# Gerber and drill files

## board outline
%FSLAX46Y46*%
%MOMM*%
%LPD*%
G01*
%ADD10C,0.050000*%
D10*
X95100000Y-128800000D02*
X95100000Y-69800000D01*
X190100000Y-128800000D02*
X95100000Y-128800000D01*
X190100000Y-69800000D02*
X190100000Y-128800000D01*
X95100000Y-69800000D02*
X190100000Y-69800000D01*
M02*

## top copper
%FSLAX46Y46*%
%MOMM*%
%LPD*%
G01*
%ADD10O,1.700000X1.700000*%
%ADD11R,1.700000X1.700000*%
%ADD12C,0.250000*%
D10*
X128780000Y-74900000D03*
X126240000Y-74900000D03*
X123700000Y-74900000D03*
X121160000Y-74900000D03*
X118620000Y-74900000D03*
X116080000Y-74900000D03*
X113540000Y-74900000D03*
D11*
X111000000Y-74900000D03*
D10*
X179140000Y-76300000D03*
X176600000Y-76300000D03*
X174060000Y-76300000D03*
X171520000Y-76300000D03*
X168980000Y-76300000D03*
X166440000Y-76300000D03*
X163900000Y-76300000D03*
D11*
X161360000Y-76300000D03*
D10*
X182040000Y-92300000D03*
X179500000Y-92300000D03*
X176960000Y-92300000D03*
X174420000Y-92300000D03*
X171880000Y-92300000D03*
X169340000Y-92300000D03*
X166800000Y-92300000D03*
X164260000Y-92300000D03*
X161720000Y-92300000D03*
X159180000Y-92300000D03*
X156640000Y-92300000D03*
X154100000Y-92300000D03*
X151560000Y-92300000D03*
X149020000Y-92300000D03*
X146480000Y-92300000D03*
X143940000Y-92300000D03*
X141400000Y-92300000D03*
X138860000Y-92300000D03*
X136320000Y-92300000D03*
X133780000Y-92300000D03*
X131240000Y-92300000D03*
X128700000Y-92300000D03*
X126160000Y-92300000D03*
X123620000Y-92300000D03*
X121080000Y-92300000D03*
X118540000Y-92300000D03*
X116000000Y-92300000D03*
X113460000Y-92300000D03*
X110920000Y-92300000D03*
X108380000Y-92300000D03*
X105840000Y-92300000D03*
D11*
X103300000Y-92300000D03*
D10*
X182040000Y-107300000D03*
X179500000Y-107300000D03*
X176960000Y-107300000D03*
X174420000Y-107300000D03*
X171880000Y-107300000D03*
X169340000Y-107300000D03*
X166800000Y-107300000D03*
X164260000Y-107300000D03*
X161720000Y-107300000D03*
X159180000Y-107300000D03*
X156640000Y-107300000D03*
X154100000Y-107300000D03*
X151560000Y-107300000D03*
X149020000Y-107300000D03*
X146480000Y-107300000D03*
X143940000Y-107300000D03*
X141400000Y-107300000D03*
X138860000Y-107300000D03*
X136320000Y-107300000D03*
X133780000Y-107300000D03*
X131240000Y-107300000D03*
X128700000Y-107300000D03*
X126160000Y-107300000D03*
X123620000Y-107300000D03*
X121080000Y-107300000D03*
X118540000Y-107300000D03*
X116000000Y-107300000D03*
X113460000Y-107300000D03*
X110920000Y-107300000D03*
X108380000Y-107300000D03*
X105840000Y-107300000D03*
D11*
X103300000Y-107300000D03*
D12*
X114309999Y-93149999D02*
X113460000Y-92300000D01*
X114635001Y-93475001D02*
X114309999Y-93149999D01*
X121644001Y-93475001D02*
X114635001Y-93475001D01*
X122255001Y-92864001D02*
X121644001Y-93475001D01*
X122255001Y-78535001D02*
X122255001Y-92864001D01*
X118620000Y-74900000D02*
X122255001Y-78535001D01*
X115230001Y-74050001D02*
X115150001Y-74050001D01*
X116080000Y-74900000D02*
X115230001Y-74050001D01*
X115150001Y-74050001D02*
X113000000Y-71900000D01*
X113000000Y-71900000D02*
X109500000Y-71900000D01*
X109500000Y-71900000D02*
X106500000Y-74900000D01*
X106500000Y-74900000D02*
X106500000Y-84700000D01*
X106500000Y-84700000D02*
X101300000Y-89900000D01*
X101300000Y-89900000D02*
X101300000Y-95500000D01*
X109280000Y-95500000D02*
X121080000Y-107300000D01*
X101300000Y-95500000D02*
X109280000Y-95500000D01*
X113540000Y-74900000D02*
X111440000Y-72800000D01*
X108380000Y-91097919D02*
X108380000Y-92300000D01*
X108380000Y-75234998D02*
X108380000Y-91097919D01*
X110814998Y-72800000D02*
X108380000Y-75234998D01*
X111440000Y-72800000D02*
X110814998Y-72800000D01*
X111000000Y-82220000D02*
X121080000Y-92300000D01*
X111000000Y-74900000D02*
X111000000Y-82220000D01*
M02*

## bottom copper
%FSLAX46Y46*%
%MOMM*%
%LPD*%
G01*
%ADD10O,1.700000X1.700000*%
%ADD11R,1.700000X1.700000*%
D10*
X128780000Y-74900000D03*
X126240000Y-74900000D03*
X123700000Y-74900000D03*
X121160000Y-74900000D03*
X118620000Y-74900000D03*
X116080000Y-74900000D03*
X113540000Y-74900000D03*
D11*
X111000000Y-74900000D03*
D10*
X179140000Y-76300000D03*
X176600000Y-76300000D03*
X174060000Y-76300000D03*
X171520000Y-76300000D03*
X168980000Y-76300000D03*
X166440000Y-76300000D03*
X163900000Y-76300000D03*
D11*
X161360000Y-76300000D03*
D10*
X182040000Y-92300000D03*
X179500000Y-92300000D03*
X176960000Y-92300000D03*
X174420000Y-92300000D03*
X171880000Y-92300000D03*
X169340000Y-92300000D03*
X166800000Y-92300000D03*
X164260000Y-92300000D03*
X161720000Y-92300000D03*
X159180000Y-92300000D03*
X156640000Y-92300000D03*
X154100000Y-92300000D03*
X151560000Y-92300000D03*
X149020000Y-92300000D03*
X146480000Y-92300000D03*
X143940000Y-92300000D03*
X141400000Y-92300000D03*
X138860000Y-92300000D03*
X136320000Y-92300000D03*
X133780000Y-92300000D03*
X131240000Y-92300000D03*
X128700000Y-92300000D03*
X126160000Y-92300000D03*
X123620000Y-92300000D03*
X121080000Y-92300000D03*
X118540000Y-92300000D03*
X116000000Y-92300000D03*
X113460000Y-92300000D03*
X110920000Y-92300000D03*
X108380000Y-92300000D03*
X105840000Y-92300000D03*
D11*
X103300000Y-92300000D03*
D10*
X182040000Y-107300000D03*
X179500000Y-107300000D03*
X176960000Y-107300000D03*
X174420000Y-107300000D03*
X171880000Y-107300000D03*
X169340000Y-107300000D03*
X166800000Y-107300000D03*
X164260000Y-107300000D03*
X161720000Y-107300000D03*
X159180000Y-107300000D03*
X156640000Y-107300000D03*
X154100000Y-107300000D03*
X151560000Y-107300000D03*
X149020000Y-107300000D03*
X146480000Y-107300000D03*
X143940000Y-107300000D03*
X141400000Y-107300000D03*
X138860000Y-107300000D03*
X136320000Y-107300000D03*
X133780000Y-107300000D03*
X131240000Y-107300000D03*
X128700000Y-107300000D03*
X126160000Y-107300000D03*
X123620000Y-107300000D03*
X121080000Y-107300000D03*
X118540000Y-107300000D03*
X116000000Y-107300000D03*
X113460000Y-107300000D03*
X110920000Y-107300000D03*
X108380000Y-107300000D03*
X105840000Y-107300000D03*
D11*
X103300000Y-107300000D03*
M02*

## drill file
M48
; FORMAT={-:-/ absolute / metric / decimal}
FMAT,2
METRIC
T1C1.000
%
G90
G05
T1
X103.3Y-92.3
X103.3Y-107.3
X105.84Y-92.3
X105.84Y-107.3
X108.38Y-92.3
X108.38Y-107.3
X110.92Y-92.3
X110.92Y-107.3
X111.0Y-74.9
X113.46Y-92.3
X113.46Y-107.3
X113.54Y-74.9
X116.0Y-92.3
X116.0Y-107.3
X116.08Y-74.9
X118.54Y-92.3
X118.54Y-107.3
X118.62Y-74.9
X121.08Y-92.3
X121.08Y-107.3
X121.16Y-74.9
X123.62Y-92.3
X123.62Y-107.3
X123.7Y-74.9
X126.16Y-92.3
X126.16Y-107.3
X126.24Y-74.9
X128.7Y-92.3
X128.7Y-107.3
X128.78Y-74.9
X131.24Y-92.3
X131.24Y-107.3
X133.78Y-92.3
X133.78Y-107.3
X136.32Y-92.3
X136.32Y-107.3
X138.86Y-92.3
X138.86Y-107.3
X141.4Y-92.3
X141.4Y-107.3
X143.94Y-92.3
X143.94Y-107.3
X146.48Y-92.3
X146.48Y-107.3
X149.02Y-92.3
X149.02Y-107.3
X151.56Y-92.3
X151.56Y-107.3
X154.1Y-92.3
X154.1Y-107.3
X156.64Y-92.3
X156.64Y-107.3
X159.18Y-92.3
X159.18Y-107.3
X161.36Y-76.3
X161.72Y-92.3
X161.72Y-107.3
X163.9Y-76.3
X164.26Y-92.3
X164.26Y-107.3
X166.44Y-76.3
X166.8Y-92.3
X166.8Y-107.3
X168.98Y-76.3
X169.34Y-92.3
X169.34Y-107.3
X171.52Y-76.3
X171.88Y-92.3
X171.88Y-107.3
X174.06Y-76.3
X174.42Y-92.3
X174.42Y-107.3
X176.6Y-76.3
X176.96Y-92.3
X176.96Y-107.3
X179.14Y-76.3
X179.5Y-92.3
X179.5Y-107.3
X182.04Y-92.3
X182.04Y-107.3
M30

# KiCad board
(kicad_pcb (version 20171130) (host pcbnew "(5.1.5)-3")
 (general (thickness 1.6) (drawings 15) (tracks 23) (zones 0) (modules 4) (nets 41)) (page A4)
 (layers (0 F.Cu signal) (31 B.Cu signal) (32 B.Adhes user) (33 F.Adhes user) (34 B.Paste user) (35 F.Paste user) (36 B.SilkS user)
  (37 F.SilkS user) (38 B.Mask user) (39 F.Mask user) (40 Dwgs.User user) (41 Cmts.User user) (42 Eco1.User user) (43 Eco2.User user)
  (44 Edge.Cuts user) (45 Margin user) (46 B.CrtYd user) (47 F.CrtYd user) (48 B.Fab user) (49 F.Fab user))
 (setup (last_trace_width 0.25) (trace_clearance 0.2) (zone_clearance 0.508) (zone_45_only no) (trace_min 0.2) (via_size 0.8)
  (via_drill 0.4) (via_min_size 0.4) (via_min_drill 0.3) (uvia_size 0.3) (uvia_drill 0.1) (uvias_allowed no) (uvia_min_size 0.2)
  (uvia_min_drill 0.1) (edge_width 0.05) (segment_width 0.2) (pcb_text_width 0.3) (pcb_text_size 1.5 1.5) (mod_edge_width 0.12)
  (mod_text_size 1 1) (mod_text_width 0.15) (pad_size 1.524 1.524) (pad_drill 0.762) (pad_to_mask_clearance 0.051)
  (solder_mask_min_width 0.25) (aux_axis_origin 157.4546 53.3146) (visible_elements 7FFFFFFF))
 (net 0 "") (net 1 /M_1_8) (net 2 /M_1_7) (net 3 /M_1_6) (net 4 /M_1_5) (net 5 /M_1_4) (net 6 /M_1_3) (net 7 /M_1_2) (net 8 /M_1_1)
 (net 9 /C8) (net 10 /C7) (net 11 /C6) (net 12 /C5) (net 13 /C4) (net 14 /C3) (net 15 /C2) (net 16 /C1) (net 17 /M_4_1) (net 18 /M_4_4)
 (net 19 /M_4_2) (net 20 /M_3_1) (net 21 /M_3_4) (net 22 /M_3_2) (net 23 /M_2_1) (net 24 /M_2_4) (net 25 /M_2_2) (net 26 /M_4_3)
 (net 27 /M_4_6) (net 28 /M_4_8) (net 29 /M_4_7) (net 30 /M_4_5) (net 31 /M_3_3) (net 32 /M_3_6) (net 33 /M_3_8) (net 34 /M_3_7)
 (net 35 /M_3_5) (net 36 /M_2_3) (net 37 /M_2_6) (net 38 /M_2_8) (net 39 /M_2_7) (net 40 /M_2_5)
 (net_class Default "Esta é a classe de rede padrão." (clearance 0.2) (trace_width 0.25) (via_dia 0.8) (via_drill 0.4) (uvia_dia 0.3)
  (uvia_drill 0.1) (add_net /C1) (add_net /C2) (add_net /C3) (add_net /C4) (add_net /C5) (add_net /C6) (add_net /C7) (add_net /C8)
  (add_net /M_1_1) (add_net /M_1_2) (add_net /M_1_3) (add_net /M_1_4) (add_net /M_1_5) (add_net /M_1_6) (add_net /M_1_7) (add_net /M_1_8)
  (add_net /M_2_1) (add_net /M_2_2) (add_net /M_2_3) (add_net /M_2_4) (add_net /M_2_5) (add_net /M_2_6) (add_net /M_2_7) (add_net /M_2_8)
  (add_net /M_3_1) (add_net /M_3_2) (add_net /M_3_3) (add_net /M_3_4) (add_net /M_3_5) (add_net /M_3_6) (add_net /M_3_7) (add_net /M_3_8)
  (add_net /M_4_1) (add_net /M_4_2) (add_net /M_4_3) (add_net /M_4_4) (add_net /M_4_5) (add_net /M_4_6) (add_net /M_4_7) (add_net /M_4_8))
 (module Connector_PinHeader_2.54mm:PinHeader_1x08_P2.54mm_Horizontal (layer F.Cu) (at 111 74.9 90)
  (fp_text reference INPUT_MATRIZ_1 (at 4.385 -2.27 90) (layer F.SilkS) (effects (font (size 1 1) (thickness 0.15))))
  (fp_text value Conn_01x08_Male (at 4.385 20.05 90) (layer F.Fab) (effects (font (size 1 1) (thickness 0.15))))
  (pad 8 thru_hole oval (at 0 17.78 90) (size 1.7 1.7) (drill 1) (layers *.Cu *.Mask) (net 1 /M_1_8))
  (pad 7 thru_hole oval (at 0 15.24 90) (size 1.7 1.7) (drill 1) (layers *.Cu *.Mask) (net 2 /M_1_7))
  (pad 6 thru_hole oval (at 0 12.7 90) (size 1.7 1.7) (drill 1) (layers *.Cu *.Mask) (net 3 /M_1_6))
  (pad 5 thru_hole oval (at 0 10.16 90) (size 1.7 1.7) (drill 1) (layers *.Cu *.Mask) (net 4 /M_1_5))
  (pad 4 thru_hole oval (at 0 7.62 90) (size 1.7 1.7) (drill 1) (layers *.Cu *.Mask) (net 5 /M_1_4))
  (pad 3 thru_hole oval (at 0 5.08 90) (size 1.7 1.7) (drill 1) (layers *.Cu *.Mask) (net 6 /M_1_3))
  (pad 2 thru_hole oval (at 0 2.54 90) (size 1.7 1.7) (drill 1) (layers *.Cu *.Mask) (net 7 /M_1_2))
  (pad 1 thru_hole rect (at 0 0 90) (size 1.7 1.7) (drill 1) (layers *.Cu *.Mask) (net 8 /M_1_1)))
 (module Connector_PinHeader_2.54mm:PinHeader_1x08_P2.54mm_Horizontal (layer F.Cu) (at 161.36 76.3 90)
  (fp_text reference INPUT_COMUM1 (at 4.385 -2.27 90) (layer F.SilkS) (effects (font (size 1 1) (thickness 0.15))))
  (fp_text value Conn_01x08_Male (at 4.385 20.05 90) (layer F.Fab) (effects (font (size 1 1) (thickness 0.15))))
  (pad 8 thru_hole oval (at 0 17.78 90) (size 1.7 1.7) (drill 1) (layers *.Cu *.Mask) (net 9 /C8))
  (pad 7 thru_hole oval (at 0 15.24 90) (size 1.7 1.7) (drill 1) (layers *.Cu *.Mask) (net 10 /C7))
  (pad 6 thru_hole oval (at 0 12.7 90) (size 1.7 1.7) (drill 1) (layers *.Cu *.Mask) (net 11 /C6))
  (pad 5 thru_hole oval (at 0 10.16 90) (size 1.7 1.7) (drill 1) (layers *.Cu *.Mask) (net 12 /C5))
  (pad 4 thru_hole oval (at 0 7.62 90) (size 1.7 1.7) (drill 1) (layers *.Cu *.Mask) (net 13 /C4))
  (pad 3 thru_hole oval (at 0 5.08 90) (size 1.7 1.7) (drill 1) (layers *.Cu *.Mask) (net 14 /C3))
  (pad 2 thru_hole oval (at 0 2.54 90) (size 1.7 1.7) (drill 1) (layers *.Cu *.Mask) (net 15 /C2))
  (pad 1 thru_hole rect (at 0 0 90) (size 1.7 1.7) (drill 1) (layers *.Cu *.Mask) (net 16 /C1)))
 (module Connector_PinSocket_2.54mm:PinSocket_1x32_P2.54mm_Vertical (layer F.Cu) (at 103.3 92.3 90)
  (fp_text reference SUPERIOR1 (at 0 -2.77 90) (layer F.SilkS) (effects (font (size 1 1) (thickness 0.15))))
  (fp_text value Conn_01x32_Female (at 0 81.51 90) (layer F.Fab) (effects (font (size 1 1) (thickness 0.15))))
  (pad 32 thru_hole oval (at 0 78.74 90) (size 1.7 1.7) (drill 1) (layers *.Cu *.Mask) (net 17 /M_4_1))
  (pad 31 thru_hole oval (at 0 76.2 90) (size 1.7 1.7) (drill 1) (layers *.Cu *.Mask) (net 13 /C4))
  (pad 30 thru_hole oval (at 0 73.66 90) (size 1.7 1.7) (drill 1) (layers *.Cu *.Mask) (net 11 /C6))
  (pad 29 thru_hole oval (at 0 71.12 90) (size 1.7 1.7) (drill 1) (layers *.Cu *.Mask) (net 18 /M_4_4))
  (pad 28 thru_hole oval (at 0 68.58 90) (size 1.7 1.7) (drill 1) (layers *.Cu *.Mask) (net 16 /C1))
  (pad 27 thru_hole oval (at 0 66.04 90) (size 1.7 1.7) (drill 1) (layers *.Cu *.Mask) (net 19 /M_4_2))
  (pad 26 thru_hole oval (at 0 63.5 90) (size 1.7 1.7) (drill 1) (layers *.Cu *.Mask) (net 9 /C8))
  (pad 25 thru_hole oval (at 0 60.96 90) (size 1.7 1.7) (drill 1) (layers *.Cu *.Mask) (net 10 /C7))
  (pad 24 thru_hole oval (at 0 58.42 90) (size 1.7 1.7) (drill 1) (layers *.Cu *.Mask) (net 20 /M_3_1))
  (pad 23 thru_hole oval (at 0 55.88 90) (size 1.7 1.7) (drill 1) (layers *.Cu *.Mask) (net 13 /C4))
  (pad 22 thru_hole oval (at 0 53.34 90) (size 1.7 1.7) (drill 1) (layers *.Cu *.Mask) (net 11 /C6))
  (pad 21 thru_hole oval (at 0 50.8 90) (size 1.7 1.7) (drill 1) (layers *.Cu *.Mask) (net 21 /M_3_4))
  (pad 20 thru_hole oval (at 0 48.26 90) (size 1.7 1.7) (drill 1) (layers *.Cu *.Mask) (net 16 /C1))
  (pad 19 thru_hole oval (at 0 45.72 90) (size 1.7 1.7) (drill 1) (layers *.Cu *.Mask) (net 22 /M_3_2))
  (pad 18 thru_hole oval (at 0 43.18 90) (size 1.7 1.7) (drill 1) (layers *.Cu *.Mask) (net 9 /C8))
  (pad 17 thru_hole oval (at 0 40.64 90) (size 1.7 1.7) (drill 1) (layers *.Cu *.Mask) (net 10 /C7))
  (pad 16 thru_hole oval (at 0 38.1 90) (size 1.7 1.7) (drill 1) (layers *.Cu *.Mask) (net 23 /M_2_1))
  (pad 15 thru_hole oval (at 0 35.56 90) (size 1.7 1.7) (drill 1) (layers *.Cu *.Mask) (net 13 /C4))
  (pad 14 thru_hole oval (at 0 33.02 90) (size 1.7 1.7) (drill 1) (layers *.Cu *.Mask) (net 11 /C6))
  (pad 13 thru_hole oval (at 0 30.48 90) (size 1.7 1.7) (drill 1) (layers *.Cu *.Mask) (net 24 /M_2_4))
  (pad 12 thru_hole oval (at 0 27.94 90) (size 1.7 1.7) (drill 1) (layers *.Cu *.Mask) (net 16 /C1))
  (pad 11 thru_hole oval (at 0 25.4 90) (size 1.7 1.7) (drill 1) (layers *.Cu *.Mask) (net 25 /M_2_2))
  (pad 10 thru_hole oval (at 0 22.86 90) (size 1.7 1.7) (drill 1) (layers *.Cu *.Mask) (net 9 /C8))
  (pad 9 thru_hole oval (at 0 20.32 90) (size 1.7 1.7) (drill 1) (layers *.Cu *.Mask) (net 10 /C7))
  (pad 8 thru_hole oval (at 0 17.78 90) (size 1.7 1.7) (drill 1) (layers *.Cu *.Mask) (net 8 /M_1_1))
  (pad 7 thru_hole oval (at 0 15.24 90) (size 1.7 1.7) (drill 1) (layers *.Cu *.Mask) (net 13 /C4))
  (pad 6 thru_hole oval (at 0 12.7 90) (size 1.7 1.7) (drill 1) (layers *.Cu *.Mask) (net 11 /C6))
  (pad 5 thru_hole oval (at 0 10.16 90) (size 1.7 1.7) (drill 1) (layers *.Cu *.Mask) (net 5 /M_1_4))
  (pad 4 thru_hole oval (at 0 7.62 90) (size 1.7 1.7) (drill 1) (layers *.Cu *.Mask) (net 16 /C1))
  (pad 3 thru_hole oval (at 0 5.08 90) (size 1.7 1.7) (drill 1) (layers *.Cu *.Mask) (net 7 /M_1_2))
  (pad 2 thru_hole oval (at 0 2.54 90) (size 1.7 1.7) (drill 1) (layers *.Cu *.Mask) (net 9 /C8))
  (pad 1 thru_hole rect (at 0 0 90) (size 1.7 1.7) (drill 1) (layers *.Cu *.Mask) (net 10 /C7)))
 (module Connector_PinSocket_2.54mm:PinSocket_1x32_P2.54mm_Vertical (layer F.Cu) (at 103.3 107.3 90)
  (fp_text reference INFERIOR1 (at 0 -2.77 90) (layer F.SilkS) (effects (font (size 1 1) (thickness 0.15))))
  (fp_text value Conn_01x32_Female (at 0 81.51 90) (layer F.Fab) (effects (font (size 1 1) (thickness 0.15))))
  (pad 32 thru_hole oval (at 0 78.74 90) (size 1.7 1.7) (drill 1) (layers *.Cu *.Mask) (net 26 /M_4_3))
  (pad 31 thru_hole oval (at 0 76.2 90) (size 1.7 1.7) (drill 1) (layers *.Cu *.Mask) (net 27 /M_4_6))
  (pad 30 thru_hole oval (at 0 73.66 90) (size 1.7 1.7) (drill 1) (layers *.Cu *.Mask) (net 12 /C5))
  (pad 29 thru_hole oval (at 0 71.12 90) (size 1.7 1.7) (drill 1) (layers *.Cu *.Mask) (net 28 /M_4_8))
  (pad 28 thru_hole oval (at 0 68.58 90) (size 1.7 1.7) (drill 1) (layers *.Cu *.Mask) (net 14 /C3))
  (pad 27 thru_hole oval (at 0 66.04 90) (size 1.7 1.7) (drill 1) (layers *.Cu *.Mask) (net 15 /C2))
  (pad 26 thru_hole oval (at 0 63.5 90) (size 1.7 1.7) (drill 1) (layers *.Cu *.Mask) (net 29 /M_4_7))
  (pad 25 thru_hole oval (at 0 60.96 90) (size 1.7 1.7) (drill 1) (layers *.Cu *.Mask) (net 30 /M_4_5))
  (pad 24 thru_hole oval (at 0 58.42 90) (size 1.7 1.7) (drill 1) (layers *.Cu *.Mask) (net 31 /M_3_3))
  (pad 23 thru_hole oval (at 0 55.88 90) (size 1.7 1.7) (drill 1) (layers *.Cu *.Mask) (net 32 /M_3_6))
  (pad 22 thru_hole oval (at 0 53.34 90) (size 1.7 1.7) (drill 1) (layers *.Cu *.Mask) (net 12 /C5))
  (pad 21 thru_hole oval (at 0 50.8 90) (size 1.7 1.7) (drill 1) (layers *.Cu *.Mask) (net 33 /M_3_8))
  (pad 20 thru_hole oval (at 0 48.26 90) (size 1.7 1.7) (drill 1) (layers *.Cu *.Mask) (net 14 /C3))
  (pad 19 thru_hole oval (at 0 45.72 90) (size 1.7 1.7) (drill 1) (layers *.Cu *.Mask) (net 15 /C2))
  (pad 18 thru_hole oval (at 0 43.18 90) (size 1.7 1.7) (drill 1) (layers *.Cu *.Mask) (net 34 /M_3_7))
  (pad 17 thru_hole oval (at 0 40.64 90) (size 1.7 1.7) (drill 1) (layers *.Cu *.Mask) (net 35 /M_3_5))
  (pad 16 thru_hole oval (at 0 38.1 90) (size 1.7 1.7) (drill 1) (layers *.Cu *.Mask) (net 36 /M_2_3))
  (pad 15 thru_hole oval (at 0 35.56 90) (size 1.7 1.7) (drill 1) (layers *.Cu *.Mask) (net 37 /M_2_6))
  (pad 14 thru_hole oval (at 0 33.02 90) (size 1.7 1.7) (drill 1) (layers *.Cu *.Mask) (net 12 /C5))
  (pad 13 thru_hole oval (at 0 30.48 90) (size 1.7 1.7) (drill 1) (layers *.Cu *.Mask) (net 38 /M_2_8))
  (pad 12 thru_hole oval (at 0 27.94 90) (size 1.7 1.7) (drill 1) (layers *.Cu *.Mask) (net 14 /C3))
  (pad 11 thru_hole oval (at 0 25.4 90) (size 1.7 1.7) (drill 1) (layers *.Cu *.Mask) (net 15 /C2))
  (pad 10 thru_hole oval (at 0 22.86 90) (size 1.7 1.7) (drill 1) (layers *.Cu *.Mask) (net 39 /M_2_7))
  (pad 9 thru_hole oval (at 0 20.32 90) (size 1.7 1.7) (drill 1) (layers *.Cu *.Mask) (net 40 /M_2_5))
  (pad 8 thru_hole oval (at 0 17.78 90) (size 1.7 1.7) (drill 1) (layers *.Cu *.Mask) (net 6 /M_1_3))
  (pad 7 thru_hole oval (at 0 15.24 90) (size 1.7 1.7) (drill 1) (layers *.Cu *.Mask) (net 3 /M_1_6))
  (pad 6 thru_hole oval (at 0 12.7 90) (size 1.7 1.7) (drill 1) (layers *.Cu *.Mask) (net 12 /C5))
  (pad 5 thru_hole oval (at 0 10.16 90) (size 1.7 1.7) (drill 1) (layers *.Cu *.Mask) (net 1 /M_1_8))
  (pad 4 thru_hole oval (at 0 7.62 90) (size 1.7 1.7) (drill 1) (layers *.Cu *.Mask) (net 14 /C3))
  (pad 3 thru_hole oval (at 0 5.08 90) (size 1.7 1.7) (drill 1) (layers *.Cu *.Mask) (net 15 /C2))
  (pad 2 thru_hole oval (at 0 2.54 90) (size 1.7 1.7) (drill 1) (layers *.Cu *.Mask) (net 2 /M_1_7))
  (pad 1 thru_hole rect (at 0 0 90) (size 1.7 1.7) (drill 1) (layers *.Cu *.Mask) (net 4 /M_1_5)))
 (gr_line (start 95.1 128.8) (end 95.1 69.8) (layer Edge.Cuts) (width 0.05))
 (gr_line (start 190.1 128.8) (end 95.1 128.8) (layer Edge.Cuts) (width 0.05))
 (gr_line (start 190.1 69.8) (end 190.1 128.8) (layer Edge.Cuts) (width 0.05))
 (gr_line (start 95.1 69.8) (end 190.1 69.8) (layer Edge.Cuts) (width 0.05))
 (segment (start 114.309999 93.149999) (end 113.46 92.3) (width 0.25) (layer F.Cu) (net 5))
 (segment (start 114.635001 93.475001) (end 114.309999 93.149999) (width 0.25) (layer F.Cu) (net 5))
 (segment (start 121.644001 93.475001) (end 114.635001 93.475001) (width 0.25) (layer F.Cu) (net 5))
 (segment (start 122.255001 92.864001) (end 121.644001 93.475001) (width 0.25) (layer F.Cu) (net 5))
 (segment (start 122.255001 78.535001) (end 122.255001 92.864001) (width 0.25) (layer F.Cu) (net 5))
 (segment (start 118.62 74.9) (end 122.255001 78.535001) (width 0.25) (layer F.Cu) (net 5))
 (segment (start 115.230001 74.050001) (end 115.150001 74.050001) (width 0.25) (layer F.Cu) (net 6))
 (segment (start 116.08 74.9) (end 115.230001 74.050001) (width 0.25) (layer F.Cu) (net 6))
 (segment (start 115.150001 74.050001) (end 113 71.9) (width 0.25) (layer F.Cu) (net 6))
 (segment (start 113 71.9) (end 109.5 71.9) (width 0.25) (layer F.Cu) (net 6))
 (segment (start 109.5 71.9) (end 106.5 74.9) (width 0.25) (layer F.Cu) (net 6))
 (segment (start 106.5 74.9) (end 106.5 84.7) (width 0.25) (layer F.Cu) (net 6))
 (segment (start 106.5 84.7) (end 101.3 89.9) (width 0.25) (layer F.Cu) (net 6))
 (segment (start 101.3 89.9) (end 101.3 95.5) (width 0.25) (layer F.Cu) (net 6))
 (segment (start 109.28 95.5) (end 121.08 107.3) (width 0.25) (layer F.Cu) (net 6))
 (segment (start 101.3 95.5) (end 109.28 95.5) (width 0.25) (layer F.Cu) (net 6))
 (segment (start 113.54 74.9) (end 111.44 72.8) (width 0.25) (layer F.Cu) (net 7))
 (segment (start 108.38 91.097919) (end 108.38 92.3) (width 0.25) (layer F.Cu) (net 7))
 (segment (start 108.38 75.234998) (end 108.38 91.097919) (width 0.25) (layer F.Cu) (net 7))
 (segment (start 110.814998 72.8) (end 108.38 75.234998) (width 0.25) (layer F.Cu) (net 7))
 (segment (start 111.44 72.8) (end 110.814998 72.8) (width 0.25) (layer F.Cu) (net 7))
 (segment (start 111 82.22) (end 121.08 92.3) (width 0.25) (layer F.Cu) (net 8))
 (segment (start 111 74.9) (end 111 82.22) (width 0.25) (layer F.Cu) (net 8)))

